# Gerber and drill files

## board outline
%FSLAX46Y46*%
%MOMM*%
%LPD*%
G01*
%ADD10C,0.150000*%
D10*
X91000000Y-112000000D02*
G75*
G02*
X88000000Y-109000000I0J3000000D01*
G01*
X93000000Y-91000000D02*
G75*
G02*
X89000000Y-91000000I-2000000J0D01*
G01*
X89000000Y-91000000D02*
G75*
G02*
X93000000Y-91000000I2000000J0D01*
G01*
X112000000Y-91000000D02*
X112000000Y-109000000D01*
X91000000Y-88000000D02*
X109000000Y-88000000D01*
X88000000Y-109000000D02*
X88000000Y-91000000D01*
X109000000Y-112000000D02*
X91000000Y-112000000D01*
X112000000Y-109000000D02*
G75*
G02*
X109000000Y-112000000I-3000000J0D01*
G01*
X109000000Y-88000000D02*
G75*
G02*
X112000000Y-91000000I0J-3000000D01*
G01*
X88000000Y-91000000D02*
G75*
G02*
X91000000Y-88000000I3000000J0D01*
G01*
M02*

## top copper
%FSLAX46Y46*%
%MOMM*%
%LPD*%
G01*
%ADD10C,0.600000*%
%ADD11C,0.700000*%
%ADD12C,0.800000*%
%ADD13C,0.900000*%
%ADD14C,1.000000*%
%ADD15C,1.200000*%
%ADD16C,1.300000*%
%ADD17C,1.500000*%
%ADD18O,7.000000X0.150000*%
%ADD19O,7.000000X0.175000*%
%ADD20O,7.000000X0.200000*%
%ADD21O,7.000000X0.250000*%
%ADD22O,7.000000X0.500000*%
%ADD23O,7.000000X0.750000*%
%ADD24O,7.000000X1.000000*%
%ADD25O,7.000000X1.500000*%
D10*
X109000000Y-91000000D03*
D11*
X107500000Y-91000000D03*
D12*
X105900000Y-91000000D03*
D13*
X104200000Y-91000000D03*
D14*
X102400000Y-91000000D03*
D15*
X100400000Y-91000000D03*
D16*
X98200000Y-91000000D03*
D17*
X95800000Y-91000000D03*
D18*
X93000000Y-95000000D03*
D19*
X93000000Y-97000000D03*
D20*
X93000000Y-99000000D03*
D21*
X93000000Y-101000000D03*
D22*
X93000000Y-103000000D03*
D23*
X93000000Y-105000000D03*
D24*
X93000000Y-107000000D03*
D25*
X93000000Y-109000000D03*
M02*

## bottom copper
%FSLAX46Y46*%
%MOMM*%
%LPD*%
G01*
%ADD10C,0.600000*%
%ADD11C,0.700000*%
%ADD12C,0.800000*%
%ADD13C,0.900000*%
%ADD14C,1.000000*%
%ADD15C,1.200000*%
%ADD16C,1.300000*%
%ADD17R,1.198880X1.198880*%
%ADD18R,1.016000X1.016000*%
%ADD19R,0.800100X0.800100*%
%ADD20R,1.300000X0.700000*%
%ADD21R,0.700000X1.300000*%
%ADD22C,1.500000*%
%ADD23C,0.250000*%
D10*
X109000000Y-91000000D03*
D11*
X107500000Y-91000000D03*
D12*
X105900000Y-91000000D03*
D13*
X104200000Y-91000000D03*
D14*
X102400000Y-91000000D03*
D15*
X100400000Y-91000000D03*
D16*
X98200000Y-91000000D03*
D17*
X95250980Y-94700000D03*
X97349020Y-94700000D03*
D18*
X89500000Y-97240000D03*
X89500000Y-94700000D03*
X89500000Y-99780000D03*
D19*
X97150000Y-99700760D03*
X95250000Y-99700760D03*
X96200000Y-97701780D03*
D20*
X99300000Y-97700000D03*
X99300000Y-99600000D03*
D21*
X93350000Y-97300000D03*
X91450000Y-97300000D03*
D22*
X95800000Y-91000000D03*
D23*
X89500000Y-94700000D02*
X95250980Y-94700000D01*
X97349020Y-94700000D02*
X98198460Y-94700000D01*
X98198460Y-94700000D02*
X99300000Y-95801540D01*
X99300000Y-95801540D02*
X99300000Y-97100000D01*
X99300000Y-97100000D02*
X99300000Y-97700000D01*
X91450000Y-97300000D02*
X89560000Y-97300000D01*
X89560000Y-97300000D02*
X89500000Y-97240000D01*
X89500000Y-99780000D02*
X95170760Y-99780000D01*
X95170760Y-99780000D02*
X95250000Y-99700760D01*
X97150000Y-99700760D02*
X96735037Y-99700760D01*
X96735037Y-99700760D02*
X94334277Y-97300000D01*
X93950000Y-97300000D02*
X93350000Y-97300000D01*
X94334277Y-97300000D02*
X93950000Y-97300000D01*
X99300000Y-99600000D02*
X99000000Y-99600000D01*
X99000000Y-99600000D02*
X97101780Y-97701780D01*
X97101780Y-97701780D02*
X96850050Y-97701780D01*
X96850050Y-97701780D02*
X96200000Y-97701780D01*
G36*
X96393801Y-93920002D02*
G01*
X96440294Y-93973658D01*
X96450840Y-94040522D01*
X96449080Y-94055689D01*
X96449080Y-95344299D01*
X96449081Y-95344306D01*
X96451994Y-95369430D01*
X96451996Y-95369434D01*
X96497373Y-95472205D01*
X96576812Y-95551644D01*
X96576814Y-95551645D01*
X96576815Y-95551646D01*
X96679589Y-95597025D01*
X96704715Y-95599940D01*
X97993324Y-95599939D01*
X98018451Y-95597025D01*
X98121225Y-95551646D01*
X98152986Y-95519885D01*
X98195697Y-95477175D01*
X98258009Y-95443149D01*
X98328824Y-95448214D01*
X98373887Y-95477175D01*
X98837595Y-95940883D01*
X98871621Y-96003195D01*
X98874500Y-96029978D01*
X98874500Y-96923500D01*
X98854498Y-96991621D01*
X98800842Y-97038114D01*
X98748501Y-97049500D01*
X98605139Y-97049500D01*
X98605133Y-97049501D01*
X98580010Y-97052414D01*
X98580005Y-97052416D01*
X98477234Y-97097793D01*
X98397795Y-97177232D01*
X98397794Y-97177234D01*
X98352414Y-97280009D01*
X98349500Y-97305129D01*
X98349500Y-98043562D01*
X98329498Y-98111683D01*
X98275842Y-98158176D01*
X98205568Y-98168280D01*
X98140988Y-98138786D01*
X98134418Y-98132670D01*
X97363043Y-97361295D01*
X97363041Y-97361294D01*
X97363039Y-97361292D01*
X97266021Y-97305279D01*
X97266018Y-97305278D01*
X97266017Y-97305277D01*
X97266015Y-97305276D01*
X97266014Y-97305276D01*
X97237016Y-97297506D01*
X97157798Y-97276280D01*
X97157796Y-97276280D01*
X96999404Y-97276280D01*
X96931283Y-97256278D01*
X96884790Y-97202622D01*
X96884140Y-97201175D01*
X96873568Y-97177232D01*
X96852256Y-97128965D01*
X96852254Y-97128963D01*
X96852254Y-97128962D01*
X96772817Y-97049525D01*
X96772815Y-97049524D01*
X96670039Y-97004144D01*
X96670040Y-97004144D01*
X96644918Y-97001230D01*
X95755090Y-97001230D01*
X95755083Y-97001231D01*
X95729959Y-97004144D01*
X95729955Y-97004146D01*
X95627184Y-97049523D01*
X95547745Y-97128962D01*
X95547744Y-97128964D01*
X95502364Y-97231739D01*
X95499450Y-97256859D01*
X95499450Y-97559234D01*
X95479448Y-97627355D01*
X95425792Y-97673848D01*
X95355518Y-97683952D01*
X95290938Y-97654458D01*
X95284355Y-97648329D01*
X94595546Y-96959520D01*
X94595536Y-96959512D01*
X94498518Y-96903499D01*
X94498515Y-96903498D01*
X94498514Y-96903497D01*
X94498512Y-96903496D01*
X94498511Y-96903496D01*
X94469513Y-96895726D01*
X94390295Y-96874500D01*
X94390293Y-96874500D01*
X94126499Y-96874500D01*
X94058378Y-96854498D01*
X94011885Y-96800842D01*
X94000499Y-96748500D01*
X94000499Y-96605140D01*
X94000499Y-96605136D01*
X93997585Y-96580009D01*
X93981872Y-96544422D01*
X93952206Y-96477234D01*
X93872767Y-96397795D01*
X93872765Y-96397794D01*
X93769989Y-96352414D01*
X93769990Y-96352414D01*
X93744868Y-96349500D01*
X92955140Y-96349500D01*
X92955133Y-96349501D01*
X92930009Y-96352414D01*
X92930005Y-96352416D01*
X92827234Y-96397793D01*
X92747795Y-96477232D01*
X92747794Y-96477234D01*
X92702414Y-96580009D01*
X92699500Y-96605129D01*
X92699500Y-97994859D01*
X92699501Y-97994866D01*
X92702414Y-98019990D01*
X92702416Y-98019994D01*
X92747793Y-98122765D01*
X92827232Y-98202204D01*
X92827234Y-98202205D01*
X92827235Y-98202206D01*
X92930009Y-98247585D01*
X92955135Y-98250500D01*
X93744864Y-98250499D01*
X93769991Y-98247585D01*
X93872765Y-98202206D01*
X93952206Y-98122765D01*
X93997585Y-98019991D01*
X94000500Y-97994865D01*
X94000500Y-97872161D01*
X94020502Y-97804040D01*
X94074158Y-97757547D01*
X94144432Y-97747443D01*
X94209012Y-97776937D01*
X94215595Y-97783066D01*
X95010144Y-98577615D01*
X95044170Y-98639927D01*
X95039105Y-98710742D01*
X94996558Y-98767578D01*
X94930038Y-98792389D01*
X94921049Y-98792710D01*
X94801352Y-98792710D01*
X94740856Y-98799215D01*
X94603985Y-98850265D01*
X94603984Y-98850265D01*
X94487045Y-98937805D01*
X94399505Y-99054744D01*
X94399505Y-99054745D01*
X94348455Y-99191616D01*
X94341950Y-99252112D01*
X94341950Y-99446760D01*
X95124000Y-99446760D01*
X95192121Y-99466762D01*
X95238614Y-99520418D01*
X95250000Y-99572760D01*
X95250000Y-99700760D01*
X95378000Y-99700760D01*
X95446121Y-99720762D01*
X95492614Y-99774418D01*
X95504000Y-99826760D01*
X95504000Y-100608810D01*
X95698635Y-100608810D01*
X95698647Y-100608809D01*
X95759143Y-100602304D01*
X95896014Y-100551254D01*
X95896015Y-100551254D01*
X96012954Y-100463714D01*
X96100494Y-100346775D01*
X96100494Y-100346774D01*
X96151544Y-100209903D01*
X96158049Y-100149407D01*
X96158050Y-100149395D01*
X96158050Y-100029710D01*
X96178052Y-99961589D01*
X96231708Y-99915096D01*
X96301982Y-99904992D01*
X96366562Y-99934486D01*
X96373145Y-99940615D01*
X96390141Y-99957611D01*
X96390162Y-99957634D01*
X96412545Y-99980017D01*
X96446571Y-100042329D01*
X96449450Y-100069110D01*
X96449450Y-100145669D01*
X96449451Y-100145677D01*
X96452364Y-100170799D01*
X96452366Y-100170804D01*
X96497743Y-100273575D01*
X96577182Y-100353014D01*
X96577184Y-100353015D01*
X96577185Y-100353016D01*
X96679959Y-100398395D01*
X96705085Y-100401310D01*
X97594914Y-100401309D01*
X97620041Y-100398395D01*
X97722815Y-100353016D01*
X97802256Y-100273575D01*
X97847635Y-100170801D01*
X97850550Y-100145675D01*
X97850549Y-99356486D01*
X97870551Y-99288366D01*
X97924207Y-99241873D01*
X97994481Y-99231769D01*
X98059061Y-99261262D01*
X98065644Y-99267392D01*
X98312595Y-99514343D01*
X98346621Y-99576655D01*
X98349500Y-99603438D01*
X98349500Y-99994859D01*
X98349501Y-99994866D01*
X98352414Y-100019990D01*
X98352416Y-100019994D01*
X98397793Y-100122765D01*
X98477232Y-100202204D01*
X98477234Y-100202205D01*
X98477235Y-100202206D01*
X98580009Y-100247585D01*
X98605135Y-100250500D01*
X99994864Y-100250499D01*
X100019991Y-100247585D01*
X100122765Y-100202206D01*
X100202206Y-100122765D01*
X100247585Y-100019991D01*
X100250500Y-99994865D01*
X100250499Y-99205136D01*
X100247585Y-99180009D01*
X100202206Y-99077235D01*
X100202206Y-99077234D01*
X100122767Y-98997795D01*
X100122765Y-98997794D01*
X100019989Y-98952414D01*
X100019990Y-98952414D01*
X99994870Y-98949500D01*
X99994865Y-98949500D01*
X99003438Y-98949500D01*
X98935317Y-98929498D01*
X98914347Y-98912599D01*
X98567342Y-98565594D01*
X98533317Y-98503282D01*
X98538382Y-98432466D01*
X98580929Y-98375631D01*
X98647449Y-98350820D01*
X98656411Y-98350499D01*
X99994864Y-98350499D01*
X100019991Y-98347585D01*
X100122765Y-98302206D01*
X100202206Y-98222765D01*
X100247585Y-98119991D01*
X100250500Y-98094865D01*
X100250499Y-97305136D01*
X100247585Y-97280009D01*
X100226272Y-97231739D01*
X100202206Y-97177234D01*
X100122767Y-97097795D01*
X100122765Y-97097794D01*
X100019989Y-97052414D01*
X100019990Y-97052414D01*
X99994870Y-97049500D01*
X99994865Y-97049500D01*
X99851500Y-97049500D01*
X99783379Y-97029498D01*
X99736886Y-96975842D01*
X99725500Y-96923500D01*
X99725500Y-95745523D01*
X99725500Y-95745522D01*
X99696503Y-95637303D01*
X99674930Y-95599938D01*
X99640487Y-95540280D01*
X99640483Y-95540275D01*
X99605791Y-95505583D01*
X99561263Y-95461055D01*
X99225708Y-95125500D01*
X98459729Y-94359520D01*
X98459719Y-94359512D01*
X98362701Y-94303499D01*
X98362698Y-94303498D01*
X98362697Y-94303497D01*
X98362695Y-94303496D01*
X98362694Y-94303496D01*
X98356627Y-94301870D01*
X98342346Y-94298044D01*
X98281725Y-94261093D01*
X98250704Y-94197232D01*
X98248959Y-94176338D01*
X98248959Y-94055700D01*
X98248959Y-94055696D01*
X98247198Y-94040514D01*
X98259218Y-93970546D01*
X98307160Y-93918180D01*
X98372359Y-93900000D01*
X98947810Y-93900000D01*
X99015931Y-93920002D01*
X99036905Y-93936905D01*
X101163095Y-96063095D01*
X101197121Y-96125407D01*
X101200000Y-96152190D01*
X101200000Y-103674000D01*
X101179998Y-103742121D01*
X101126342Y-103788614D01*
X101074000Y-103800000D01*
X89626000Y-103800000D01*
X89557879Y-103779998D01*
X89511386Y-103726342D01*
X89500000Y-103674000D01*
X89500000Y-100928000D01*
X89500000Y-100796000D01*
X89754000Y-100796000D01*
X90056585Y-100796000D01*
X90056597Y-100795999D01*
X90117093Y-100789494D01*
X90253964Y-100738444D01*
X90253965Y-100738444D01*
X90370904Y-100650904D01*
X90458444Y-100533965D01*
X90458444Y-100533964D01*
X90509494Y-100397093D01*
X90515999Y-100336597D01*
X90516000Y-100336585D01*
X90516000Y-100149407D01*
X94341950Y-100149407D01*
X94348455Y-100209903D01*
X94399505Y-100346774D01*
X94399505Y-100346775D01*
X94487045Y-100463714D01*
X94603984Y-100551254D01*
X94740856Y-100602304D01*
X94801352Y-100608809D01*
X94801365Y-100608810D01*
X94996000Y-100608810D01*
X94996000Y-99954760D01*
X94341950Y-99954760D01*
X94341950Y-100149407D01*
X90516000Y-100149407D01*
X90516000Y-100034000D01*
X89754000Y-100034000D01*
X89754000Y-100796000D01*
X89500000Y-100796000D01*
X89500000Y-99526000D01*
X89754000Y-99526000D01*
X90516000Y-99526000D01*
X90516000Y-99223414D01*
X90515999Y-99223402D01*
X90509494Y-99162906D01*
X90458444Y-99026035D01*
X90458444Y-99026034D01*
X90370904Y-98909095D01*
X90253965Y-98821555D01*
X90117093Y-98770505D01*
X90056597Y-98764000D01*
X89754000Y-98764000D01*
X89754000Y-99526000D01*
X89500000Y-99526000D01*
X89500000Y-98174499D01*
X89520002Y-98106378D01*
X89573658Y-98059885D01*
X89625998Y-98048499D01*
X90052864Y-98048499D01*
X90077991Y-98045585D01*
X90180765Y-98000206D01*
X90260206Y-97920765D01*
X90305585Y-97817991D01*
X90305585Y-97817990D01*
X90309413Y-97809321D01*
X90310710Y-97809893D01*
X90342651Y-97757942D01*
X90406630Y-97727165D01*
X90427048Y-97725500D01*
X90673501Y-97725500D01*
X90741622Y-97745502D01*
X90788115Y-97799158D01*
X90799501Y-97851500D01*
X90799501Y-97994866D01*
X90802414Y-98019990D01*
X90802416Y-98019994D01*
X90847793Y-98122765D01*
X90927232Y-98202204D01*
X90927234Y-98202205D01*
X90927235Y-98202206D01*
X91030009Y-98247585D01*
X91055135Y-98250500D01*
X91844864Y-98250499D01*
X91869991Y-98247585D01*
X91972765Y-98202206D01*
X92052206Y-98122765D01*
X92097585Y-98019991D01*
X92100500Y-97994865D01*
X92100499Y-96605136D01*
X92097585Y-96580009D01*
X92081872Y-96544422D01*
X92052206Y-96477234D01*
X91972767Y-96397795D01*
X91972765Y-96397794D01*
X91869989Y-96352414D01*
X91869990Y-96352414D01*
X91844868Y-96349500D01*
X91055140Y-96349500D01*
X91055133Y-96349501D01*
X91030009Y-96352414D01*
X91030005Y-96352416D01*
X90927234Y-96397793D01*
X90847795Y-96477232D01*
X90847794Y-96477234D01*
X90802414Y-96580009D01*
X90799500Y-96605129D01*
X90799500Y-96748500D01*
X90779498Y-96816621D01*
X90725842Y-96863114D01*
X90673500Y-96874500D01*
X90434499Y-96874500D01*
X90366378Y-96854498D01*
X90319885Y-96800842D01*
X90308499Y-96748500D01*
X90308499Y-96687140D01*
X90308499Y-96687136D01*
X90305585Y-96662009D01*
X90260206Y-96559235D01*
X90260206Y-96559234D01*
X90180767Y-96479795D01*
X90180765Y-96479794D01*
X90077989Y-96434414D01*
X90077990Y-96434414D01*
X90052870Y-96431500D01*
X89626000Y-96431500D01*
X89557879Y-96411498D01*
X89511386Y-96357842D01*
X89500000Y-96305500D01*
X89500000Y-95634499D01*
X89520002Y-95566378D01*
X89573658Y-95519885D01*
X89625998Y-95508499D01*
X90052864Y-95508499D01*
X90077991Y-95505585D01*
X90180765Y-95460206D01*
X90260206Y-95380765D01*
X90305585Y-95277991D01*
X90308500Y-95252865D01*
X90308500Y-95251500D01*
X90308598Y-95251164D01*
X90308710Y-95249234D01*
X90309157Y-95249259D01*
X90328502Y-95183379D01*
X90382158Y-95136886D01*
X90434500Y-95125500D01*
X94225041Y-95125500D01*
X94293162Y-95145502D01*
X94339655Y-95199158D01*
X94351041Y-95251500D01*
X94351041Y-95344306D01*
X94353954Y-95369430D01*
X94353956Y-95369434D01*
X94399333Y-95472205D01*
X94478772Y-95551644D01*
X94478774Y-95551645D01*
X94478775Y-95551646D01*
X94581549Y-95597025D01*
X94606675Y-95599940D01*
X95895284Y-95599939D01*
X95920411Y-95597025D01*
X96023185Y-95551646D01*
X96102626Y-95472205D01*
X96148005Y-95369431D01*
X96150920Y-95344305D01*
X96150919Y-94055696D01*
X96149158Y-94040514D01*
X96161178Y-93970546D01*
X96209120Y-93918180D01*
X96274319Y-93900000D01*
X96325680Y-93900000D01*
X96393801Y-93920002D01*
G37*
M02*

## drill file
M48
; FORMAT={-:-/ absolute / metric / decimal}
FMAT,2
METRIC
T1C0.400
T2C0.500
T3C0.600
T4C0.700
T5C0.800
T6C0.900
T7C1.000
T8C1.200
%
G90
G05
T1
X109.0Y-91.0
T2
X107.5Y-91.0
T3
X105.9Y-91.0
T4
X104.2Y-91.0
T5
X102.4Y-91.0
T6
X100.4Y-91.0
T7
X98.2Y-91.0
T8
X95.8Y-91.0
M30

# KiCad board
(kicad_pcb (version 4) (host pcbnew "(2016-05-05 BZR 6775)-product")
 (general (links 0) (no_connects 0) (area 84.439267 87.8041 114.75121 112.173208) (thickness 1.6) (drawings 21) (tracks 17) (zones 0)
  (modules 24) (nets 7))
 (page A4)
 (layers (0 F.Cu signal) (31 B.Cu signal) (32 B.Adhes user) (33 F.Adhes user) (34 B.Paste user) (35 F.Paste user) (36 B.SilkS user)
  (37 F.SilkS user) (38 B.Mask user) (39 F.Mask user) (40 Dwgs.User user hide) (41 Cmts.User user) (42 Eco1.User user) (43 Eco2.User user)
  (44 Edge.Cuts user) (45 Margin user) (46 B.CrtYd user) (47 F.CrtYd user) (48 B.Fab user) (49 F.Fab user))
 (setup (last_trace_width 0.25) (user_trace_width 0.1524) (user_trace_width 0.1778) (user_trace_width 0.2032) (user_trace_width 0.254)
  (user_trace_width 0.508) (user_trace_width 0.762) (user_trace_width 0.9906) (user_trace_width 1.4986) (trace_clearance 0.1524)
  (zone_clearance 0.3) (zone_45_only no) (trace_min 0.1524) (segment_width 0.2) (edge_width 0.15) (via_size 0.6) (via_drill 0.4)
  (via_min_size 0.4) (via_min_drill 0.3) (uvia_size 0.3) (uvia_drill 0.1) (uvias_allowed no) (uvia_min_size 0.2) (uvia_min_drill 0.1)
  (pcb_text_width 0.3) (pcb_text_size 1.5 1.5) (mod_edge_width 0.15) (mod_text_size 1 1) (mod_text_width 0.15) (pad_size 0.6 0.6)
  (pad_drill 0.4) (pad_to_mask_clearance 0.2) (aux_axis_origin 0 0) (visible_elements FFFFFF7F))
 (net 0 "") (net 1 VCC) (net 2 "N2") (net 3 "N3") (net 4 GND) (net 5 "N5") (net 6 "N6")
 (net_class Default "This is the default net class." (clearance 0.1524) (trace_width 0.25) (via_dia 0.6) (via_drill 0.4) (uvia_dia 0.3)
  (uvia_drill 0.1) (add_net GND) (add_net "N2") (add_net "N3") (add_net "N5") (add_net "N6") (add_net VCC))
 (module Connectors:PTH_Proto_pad (layer F.Cu) (at 109 91)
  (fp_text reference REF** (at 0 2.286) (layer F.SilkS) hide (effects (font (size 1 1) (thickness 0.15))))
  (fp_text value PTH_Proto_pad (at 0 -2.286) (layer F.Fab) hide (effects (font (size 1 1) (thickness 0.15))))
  (pad 1 thru_hole circle (at 0 0) (size 0.6 0.6) (drill 0.4) (layers *.Cu *.Mask F.SilkS)))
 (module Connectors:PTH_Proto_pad (layer F.Cu) (at 107.5 91)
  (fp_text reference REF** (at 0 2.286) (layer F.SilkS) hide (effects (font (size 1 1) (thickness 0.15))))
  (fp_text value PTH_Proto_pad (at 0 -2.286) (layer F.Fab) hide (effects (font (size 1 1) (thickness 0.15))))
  (pad 1 thru_hole circle (at 0 0) (size 0.7 0.7) (drill 0.5) (layers *.Cu *.Mask F.SilkS)))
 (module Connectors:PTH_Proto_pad (layer F.Cu) (at 105.9 91)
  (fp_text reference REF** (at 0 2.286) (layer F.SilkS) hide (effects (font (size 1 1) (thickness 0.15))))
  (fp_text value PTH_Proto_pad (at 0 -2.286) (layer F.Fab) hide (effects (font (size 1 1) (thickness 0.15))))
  (pad 1 thru_hole circle (at 0 0) (size 0.8 0.8) (drill 0.6) (layers *.Cu *.Mask F.SilkS)))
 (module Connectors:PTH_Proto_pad (layer F.Cu) (at 104.2 91)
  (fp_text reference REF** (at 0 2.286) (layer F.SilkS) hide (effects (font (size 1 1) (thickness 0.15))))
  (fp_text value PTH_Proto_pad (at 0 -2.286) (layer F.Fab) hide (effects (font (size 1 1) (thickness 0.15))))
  (pad 1 thru_hole circle (at 0 0) (size 0.9 0.9) (drill 0.7) (layers *.Cu *.Mask F.SilkS)))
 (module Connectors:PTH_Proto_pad (layer F.Cu) (at 102.4 91)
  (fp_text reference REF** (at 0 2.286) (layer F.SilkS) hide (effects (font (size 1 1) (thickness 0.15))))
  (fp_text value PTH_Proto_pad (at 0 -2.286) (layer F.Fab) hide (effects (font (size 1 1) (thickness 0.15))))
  (pad 1 thru_hole circle (at 0 0) (size 1 1) (drill 0.8) (layers *.Cu *.Mask F.SilkS)))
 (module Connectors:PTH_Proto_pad (layer F.Cu) (at 100.4 91)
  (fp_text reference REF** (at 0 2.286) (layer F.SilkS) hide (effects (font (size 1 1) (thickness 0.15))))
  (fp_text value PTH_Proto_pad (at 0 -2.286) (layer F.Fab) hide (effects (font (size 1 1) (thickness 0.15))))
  (pad 1 thru_hole circle (at 0 0) (size 1.2 1.2) (drill 0.9) (layers *.Cu *.Mask F.SilkS)))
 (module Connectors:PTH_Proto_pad (layer F.Cu) (at 98.2 91)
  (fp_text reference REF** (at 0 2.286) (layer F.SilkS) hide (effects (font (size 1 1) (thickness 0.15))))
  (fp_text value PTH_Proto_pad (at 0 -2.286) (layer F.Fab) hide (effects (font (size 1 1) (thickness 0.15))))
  (pad 1 thru_hole circle (at 0 0) (size 1.3 1.3) (drill 1) (layers *.Cu *.Mask F.SilkS)))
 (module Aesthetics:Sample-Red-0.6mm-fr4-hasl (layer B.Cu) (at 100 102.6 180)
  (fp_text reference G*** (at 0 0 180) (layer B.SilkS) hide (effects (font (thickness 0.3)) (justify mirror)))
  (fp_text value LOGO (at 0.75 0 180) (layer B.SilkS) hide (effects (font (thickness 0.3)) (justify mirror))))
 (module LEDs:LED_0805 (layer B.Cu) (at 96.3 94.7 180)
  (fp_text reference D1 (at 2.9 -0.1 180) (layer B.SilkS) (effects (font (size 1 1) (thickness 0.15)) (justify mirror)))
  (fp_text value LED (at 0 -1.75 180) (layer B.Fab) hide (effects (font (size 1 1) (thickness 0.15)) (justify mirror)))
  (pad 2 smd rect (at 1.04902 0) (size 1.19888 1.19888) (layers B.Cu B.Paste B.Mask) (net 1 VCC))
  (pad 1 smd rect (at -1.04902 0) (size 1.19888 1.19888) (layers B.Cu B.Paste B.Mask) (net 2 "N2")))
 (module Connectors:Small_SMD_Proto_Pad (layer B.Cu) (at 89.5 97.24)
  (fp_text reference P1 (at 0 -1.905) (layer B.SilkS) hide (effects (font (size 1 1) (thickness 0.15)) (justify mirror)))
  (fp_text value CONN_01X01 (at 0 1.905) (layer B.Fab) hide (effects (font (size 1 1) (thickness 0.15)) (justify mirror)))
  (pad 1 smd rect (at 0 0) (size 1.016 1.016) (layers B.Cu B.Paste B.Mask) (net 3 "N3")))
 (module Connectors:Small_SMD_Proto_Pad (layer B.Cu) (at 89.5 94.7)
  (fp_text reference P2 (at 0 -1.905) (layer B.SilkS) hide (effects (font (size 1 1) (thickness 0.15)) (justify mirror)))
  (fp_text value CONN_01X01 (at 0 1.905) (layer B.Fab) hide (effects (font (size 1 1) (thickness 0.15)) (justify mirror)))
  (pad 1 smd rect (at 0 0) (size 1.016 1.016) (layers B.Cu B.Paste B.Mask) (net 1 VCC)))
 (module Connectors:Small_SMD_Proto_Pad (layer B.Cu) (at 89.5 99.78)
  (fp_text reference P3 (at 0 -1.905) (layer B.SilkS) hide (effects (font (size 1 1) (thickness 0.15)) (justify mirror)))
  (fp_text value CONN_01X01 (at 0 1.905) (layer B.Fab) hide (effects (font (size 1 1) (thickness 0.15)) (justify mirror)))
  (pad 1 smd rect (at 0 0) (size 1.016 1.016) (layers B.Cu B.Paste B.Mask) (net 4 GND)))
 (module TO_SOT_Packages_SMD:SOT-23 (layer B.Cu) (at 96.2 98.7 180)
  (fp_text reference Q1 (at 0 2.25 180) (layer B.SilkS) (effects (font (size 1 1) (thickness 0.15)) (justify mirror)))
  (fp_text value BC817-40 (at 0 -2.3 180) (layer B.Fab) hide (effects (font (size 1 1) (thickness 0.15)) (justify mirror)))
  (pad 1 smd rect (at -0.95 -1.00076 180) (size 0.8001 0.8001) (layers B.Cu B.Paste B.Mask) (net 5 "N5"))
  (pad 2 smd rect (at 0.95 -1.00076 180) (size 0.8001 0.8001) (layers B.Cu B.Paste B.Mask) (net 4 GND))
  (pad 3 smd rect (at 0 0.99822 180) (size 0.8001 0.8001) (layers B.Cu B.Paste B.Mask) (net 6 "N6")))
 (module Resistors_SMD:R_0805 (layer B.Cu) (at 99.3 98.65 270)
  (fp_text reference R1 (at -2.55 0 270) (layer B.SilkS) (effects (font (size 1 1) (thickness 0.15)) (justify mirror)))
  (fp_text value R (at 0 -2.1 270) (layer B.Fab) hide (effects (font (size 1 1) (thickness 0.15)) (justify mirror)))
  (pad 1 smd rect (at -0.95 0 270) (size 0.7 1.3) (layers B.Cu B.Paste B.Mask) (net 2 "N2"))
  (pad 2 smd rect (at 0.95 0 270) (size 0.7 1.3) (layers B.Cu B.Paste B.Mask) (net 6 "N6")))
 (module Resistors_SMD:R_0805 (layer B.Cu) (at 92.4 97.3 180)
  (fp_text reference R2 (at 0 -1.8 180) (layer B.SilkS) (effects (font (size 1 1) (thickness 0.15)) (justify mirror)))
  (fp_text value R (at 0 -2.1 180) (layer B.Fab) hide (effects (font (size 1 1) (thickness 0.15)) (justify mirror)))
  (pad 1 smd rect (at -0.95 0 180) (size 0.7 1.3) (layers B.Cu B.Paste B.Mask) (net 5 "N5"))
  (pad 2 smd rect (at 0.95 0 180) (size 0.7 1.3) (layers B.Cu B.Paste B.Mask) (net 3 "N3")))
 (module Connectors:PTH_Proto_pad (layer F.Cu) (at 95.8 91)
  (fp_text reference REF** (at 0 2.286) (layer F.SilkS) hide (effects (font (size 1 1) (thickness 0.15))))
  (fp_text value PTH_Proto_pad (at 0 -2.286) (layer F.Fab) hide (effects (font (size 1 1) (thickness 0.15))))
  (pad 1 thru_hole circle (at 0 0) (size 1.5 1.5) (drill 1.2) (layers *.Cu *.Mask F.SilkS)))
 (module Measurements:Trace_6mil (layer F.Cu) (at 93 95)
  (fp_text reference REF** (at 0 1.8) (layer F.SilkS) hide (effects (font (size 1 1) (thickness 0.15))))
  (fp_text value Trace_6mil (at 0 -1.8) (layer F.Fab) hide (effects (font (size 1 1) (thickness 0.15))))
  (pad 1 smd oval (at 0 0) (size 7 0.15) (layers F.Cu F.Paste F.Mask)))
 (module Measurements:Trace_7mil (layer F.Cu) (at 93 97)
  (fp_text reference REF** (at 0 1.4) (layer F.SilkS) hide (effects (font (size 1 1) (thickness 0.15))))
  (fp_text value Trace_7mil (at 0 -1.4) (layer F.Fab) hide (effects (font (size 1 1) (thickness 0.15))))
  (pad 1 smd oval (at 0 0) (size 7 0.175) (layers F.Cu F.Paste F.Mask)))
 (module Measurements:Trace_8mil (layer F.Cu) (at 93 99)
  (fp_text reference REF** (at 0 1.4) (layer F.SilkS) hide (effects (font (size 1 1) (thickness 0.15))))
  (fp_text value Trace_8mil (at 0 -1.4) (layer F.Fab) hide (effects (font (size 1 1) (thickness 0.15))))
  (pad 1 smd oval (at 0 0) (size 7 0.2) (layers F.Cu F.Paste F.Mask)))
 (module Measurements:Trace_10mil (layer F.Cu) (at 93 101)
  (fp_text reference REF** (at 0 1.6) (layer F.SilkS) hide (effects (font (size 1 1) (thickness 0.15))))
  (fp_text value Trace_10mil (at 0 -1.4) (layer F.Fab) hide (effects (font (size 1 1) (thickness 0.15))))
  (pad 1 smd oval (at 0 0) (size 7 0.25) (layers F.Cu F.Paste F.Mask)))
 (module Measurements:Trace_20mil (layer F.Cu) (at 93 103)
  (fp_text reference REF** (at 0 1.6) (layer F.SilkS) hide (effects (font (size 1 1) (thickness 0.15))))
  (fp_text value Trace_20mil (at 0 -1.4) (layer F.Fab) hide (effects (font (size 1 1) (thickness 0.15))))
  (pad 1 smd oval (at 0 0) (size 7 0.5) (layers F.Cu F.Paste F.Mask)))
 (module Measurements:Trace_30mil (layer F.Cu) (at 93 105)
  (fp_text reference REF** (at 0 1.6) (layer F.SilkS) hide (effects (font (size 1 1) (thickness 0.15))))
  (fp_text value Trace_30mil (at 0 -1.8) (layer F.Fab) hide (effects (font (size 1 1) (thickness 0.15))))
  (pad 1 smd oval (at 0 0) (size 7 0.75) (layers F.Cu F.Paste F.Mask)))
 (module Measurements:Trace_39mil (layer F.Cu) (at 93 107)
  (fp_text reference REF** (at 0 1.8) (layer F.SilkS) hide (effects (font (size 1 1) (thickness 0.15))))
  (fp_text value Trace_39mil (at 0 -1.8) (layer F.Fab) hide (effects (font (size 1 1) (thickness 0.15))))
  (pad 1 smd oval (at 0 0) (size 7 1) (layers F.Cu F.Paste F.Mask)))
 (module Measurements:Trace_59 (layer F.Cu) (at 93 109)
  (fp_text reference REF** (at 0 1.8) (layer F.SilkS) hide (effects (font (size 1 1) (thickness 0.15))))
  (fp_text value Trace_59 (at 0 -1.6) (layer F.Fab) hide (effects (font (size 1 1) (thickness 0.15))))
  (pad 1 smd oval (at 0 0) (size 7 1.5) (layers F.Cu F.Paste F.Mask)))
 (gr_arc (start 91 109) (end 91 112) (angle 90) (layer Edge.Cuts) (width 0.15))
 (gr_circle (center 91 91) (end 93 91) (layer Edge.Cuts) (width 0.15))
 (gr_line (start 112 91) (end 112 109) (layer Edge.Cuts) (width 0.15))
 (gr_line (start 91 88) (end 109 88) (layer Edge.Cuts) (width 0.15))
 (gr_line (start 88 109) (end 88 91) (layer Edge.Cuts) (width 0.15))
 (gr_line (start 109 112) (end 91 112) (layer Edge.Cuts) (width 0.15))
 (gr_arc (start 109 109) (end 112 109) (angle 90) (layer Edge.Cuts) (width 0.15))
 (gr_arc (start 109 91) (end 109 88) (angle 90) (layer Edge.Cuts) (width 0.15))
 (gr_arc (start 91 91) (end 88 91) (angle 90) (layer Edge.Cuts) (width 0.15))
 (segment (start 89.5 94.7) (end 95.25098 94.7) (width 0.25) (layer B.Cu) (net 1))
 (segment (start 97.34902 94.7) (end 98.19846 94.7) (width 0.25) (layer B.Cu) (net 2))
 (segment (start 98.19846 94.7) (end 99.3 95.80154) (width 0.25) (layer B.Cu) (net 2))
 (segment (start 99.3 95.80154) (end 99.3 97.1) (width 0.25) (layer B.Cu) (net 2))
 (segment (start 99.3 97.1) (end 99.3 97.7) (width 0.25) (layer B.Cu) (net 2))
 (segment (start 91.45 97.3) (end 89.56 97.3) (width 0.25) (layer B.Cu) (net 3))
 (segment (start 89.56 97.3) (end 89.5 97.24) (width 0.25) (layer B.Cu) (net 3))
 (segment (start 89.5 99.78) (end 95.17076 99.78) (width 0.25) (layer B.Cu) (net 4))
 (segment (start 95.17076 99.78) (end 95.25 99.70076) (width 0.25) (layer B.Cu) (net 4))
 (segment (start 97.15 99.70076) (end 96.735037 99.70076) (width 0.25) (layer B.Cu) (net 5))
 (segment (start 96.735037 99.70076) (end 94.334277 97.3) (width 0.25) (layer B.Cu) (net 5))
 (segment (start 93.95 97.3) (end 93.35 97.3) (width 0.25) (layer B.Cu) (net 5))
 (segment (start 94.334277 97.3) (end 93.95 97.3) (width 0.25) (layer B.Cu) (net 5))
 (segment (start 99.3 99.6) (end 99 99.6) (width 0.25) (layer B.Cu) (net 6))
 (segment (start 99 99.6) (end 97.10178 97.70178) (width 0.25) (layer B.Cu) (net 6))
 (segment (start 97.10178 97.70178) (end 96.85005 97.70178) (width 0.25) (layer B.Cu) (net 6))
 (segment (start 96.85005 97.70178) (end 96.2 97.70178) (width 0.25) (layer B.Cu) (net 6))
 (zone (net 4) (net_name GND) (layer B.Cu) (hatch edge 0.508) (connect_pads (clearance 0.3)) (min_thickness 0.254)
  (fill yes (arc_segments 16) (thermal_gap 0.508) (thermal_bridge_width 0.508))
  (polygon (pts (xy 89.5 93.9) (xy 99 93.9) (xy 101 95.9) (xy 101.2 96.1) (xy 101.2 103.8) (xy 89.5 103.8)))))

